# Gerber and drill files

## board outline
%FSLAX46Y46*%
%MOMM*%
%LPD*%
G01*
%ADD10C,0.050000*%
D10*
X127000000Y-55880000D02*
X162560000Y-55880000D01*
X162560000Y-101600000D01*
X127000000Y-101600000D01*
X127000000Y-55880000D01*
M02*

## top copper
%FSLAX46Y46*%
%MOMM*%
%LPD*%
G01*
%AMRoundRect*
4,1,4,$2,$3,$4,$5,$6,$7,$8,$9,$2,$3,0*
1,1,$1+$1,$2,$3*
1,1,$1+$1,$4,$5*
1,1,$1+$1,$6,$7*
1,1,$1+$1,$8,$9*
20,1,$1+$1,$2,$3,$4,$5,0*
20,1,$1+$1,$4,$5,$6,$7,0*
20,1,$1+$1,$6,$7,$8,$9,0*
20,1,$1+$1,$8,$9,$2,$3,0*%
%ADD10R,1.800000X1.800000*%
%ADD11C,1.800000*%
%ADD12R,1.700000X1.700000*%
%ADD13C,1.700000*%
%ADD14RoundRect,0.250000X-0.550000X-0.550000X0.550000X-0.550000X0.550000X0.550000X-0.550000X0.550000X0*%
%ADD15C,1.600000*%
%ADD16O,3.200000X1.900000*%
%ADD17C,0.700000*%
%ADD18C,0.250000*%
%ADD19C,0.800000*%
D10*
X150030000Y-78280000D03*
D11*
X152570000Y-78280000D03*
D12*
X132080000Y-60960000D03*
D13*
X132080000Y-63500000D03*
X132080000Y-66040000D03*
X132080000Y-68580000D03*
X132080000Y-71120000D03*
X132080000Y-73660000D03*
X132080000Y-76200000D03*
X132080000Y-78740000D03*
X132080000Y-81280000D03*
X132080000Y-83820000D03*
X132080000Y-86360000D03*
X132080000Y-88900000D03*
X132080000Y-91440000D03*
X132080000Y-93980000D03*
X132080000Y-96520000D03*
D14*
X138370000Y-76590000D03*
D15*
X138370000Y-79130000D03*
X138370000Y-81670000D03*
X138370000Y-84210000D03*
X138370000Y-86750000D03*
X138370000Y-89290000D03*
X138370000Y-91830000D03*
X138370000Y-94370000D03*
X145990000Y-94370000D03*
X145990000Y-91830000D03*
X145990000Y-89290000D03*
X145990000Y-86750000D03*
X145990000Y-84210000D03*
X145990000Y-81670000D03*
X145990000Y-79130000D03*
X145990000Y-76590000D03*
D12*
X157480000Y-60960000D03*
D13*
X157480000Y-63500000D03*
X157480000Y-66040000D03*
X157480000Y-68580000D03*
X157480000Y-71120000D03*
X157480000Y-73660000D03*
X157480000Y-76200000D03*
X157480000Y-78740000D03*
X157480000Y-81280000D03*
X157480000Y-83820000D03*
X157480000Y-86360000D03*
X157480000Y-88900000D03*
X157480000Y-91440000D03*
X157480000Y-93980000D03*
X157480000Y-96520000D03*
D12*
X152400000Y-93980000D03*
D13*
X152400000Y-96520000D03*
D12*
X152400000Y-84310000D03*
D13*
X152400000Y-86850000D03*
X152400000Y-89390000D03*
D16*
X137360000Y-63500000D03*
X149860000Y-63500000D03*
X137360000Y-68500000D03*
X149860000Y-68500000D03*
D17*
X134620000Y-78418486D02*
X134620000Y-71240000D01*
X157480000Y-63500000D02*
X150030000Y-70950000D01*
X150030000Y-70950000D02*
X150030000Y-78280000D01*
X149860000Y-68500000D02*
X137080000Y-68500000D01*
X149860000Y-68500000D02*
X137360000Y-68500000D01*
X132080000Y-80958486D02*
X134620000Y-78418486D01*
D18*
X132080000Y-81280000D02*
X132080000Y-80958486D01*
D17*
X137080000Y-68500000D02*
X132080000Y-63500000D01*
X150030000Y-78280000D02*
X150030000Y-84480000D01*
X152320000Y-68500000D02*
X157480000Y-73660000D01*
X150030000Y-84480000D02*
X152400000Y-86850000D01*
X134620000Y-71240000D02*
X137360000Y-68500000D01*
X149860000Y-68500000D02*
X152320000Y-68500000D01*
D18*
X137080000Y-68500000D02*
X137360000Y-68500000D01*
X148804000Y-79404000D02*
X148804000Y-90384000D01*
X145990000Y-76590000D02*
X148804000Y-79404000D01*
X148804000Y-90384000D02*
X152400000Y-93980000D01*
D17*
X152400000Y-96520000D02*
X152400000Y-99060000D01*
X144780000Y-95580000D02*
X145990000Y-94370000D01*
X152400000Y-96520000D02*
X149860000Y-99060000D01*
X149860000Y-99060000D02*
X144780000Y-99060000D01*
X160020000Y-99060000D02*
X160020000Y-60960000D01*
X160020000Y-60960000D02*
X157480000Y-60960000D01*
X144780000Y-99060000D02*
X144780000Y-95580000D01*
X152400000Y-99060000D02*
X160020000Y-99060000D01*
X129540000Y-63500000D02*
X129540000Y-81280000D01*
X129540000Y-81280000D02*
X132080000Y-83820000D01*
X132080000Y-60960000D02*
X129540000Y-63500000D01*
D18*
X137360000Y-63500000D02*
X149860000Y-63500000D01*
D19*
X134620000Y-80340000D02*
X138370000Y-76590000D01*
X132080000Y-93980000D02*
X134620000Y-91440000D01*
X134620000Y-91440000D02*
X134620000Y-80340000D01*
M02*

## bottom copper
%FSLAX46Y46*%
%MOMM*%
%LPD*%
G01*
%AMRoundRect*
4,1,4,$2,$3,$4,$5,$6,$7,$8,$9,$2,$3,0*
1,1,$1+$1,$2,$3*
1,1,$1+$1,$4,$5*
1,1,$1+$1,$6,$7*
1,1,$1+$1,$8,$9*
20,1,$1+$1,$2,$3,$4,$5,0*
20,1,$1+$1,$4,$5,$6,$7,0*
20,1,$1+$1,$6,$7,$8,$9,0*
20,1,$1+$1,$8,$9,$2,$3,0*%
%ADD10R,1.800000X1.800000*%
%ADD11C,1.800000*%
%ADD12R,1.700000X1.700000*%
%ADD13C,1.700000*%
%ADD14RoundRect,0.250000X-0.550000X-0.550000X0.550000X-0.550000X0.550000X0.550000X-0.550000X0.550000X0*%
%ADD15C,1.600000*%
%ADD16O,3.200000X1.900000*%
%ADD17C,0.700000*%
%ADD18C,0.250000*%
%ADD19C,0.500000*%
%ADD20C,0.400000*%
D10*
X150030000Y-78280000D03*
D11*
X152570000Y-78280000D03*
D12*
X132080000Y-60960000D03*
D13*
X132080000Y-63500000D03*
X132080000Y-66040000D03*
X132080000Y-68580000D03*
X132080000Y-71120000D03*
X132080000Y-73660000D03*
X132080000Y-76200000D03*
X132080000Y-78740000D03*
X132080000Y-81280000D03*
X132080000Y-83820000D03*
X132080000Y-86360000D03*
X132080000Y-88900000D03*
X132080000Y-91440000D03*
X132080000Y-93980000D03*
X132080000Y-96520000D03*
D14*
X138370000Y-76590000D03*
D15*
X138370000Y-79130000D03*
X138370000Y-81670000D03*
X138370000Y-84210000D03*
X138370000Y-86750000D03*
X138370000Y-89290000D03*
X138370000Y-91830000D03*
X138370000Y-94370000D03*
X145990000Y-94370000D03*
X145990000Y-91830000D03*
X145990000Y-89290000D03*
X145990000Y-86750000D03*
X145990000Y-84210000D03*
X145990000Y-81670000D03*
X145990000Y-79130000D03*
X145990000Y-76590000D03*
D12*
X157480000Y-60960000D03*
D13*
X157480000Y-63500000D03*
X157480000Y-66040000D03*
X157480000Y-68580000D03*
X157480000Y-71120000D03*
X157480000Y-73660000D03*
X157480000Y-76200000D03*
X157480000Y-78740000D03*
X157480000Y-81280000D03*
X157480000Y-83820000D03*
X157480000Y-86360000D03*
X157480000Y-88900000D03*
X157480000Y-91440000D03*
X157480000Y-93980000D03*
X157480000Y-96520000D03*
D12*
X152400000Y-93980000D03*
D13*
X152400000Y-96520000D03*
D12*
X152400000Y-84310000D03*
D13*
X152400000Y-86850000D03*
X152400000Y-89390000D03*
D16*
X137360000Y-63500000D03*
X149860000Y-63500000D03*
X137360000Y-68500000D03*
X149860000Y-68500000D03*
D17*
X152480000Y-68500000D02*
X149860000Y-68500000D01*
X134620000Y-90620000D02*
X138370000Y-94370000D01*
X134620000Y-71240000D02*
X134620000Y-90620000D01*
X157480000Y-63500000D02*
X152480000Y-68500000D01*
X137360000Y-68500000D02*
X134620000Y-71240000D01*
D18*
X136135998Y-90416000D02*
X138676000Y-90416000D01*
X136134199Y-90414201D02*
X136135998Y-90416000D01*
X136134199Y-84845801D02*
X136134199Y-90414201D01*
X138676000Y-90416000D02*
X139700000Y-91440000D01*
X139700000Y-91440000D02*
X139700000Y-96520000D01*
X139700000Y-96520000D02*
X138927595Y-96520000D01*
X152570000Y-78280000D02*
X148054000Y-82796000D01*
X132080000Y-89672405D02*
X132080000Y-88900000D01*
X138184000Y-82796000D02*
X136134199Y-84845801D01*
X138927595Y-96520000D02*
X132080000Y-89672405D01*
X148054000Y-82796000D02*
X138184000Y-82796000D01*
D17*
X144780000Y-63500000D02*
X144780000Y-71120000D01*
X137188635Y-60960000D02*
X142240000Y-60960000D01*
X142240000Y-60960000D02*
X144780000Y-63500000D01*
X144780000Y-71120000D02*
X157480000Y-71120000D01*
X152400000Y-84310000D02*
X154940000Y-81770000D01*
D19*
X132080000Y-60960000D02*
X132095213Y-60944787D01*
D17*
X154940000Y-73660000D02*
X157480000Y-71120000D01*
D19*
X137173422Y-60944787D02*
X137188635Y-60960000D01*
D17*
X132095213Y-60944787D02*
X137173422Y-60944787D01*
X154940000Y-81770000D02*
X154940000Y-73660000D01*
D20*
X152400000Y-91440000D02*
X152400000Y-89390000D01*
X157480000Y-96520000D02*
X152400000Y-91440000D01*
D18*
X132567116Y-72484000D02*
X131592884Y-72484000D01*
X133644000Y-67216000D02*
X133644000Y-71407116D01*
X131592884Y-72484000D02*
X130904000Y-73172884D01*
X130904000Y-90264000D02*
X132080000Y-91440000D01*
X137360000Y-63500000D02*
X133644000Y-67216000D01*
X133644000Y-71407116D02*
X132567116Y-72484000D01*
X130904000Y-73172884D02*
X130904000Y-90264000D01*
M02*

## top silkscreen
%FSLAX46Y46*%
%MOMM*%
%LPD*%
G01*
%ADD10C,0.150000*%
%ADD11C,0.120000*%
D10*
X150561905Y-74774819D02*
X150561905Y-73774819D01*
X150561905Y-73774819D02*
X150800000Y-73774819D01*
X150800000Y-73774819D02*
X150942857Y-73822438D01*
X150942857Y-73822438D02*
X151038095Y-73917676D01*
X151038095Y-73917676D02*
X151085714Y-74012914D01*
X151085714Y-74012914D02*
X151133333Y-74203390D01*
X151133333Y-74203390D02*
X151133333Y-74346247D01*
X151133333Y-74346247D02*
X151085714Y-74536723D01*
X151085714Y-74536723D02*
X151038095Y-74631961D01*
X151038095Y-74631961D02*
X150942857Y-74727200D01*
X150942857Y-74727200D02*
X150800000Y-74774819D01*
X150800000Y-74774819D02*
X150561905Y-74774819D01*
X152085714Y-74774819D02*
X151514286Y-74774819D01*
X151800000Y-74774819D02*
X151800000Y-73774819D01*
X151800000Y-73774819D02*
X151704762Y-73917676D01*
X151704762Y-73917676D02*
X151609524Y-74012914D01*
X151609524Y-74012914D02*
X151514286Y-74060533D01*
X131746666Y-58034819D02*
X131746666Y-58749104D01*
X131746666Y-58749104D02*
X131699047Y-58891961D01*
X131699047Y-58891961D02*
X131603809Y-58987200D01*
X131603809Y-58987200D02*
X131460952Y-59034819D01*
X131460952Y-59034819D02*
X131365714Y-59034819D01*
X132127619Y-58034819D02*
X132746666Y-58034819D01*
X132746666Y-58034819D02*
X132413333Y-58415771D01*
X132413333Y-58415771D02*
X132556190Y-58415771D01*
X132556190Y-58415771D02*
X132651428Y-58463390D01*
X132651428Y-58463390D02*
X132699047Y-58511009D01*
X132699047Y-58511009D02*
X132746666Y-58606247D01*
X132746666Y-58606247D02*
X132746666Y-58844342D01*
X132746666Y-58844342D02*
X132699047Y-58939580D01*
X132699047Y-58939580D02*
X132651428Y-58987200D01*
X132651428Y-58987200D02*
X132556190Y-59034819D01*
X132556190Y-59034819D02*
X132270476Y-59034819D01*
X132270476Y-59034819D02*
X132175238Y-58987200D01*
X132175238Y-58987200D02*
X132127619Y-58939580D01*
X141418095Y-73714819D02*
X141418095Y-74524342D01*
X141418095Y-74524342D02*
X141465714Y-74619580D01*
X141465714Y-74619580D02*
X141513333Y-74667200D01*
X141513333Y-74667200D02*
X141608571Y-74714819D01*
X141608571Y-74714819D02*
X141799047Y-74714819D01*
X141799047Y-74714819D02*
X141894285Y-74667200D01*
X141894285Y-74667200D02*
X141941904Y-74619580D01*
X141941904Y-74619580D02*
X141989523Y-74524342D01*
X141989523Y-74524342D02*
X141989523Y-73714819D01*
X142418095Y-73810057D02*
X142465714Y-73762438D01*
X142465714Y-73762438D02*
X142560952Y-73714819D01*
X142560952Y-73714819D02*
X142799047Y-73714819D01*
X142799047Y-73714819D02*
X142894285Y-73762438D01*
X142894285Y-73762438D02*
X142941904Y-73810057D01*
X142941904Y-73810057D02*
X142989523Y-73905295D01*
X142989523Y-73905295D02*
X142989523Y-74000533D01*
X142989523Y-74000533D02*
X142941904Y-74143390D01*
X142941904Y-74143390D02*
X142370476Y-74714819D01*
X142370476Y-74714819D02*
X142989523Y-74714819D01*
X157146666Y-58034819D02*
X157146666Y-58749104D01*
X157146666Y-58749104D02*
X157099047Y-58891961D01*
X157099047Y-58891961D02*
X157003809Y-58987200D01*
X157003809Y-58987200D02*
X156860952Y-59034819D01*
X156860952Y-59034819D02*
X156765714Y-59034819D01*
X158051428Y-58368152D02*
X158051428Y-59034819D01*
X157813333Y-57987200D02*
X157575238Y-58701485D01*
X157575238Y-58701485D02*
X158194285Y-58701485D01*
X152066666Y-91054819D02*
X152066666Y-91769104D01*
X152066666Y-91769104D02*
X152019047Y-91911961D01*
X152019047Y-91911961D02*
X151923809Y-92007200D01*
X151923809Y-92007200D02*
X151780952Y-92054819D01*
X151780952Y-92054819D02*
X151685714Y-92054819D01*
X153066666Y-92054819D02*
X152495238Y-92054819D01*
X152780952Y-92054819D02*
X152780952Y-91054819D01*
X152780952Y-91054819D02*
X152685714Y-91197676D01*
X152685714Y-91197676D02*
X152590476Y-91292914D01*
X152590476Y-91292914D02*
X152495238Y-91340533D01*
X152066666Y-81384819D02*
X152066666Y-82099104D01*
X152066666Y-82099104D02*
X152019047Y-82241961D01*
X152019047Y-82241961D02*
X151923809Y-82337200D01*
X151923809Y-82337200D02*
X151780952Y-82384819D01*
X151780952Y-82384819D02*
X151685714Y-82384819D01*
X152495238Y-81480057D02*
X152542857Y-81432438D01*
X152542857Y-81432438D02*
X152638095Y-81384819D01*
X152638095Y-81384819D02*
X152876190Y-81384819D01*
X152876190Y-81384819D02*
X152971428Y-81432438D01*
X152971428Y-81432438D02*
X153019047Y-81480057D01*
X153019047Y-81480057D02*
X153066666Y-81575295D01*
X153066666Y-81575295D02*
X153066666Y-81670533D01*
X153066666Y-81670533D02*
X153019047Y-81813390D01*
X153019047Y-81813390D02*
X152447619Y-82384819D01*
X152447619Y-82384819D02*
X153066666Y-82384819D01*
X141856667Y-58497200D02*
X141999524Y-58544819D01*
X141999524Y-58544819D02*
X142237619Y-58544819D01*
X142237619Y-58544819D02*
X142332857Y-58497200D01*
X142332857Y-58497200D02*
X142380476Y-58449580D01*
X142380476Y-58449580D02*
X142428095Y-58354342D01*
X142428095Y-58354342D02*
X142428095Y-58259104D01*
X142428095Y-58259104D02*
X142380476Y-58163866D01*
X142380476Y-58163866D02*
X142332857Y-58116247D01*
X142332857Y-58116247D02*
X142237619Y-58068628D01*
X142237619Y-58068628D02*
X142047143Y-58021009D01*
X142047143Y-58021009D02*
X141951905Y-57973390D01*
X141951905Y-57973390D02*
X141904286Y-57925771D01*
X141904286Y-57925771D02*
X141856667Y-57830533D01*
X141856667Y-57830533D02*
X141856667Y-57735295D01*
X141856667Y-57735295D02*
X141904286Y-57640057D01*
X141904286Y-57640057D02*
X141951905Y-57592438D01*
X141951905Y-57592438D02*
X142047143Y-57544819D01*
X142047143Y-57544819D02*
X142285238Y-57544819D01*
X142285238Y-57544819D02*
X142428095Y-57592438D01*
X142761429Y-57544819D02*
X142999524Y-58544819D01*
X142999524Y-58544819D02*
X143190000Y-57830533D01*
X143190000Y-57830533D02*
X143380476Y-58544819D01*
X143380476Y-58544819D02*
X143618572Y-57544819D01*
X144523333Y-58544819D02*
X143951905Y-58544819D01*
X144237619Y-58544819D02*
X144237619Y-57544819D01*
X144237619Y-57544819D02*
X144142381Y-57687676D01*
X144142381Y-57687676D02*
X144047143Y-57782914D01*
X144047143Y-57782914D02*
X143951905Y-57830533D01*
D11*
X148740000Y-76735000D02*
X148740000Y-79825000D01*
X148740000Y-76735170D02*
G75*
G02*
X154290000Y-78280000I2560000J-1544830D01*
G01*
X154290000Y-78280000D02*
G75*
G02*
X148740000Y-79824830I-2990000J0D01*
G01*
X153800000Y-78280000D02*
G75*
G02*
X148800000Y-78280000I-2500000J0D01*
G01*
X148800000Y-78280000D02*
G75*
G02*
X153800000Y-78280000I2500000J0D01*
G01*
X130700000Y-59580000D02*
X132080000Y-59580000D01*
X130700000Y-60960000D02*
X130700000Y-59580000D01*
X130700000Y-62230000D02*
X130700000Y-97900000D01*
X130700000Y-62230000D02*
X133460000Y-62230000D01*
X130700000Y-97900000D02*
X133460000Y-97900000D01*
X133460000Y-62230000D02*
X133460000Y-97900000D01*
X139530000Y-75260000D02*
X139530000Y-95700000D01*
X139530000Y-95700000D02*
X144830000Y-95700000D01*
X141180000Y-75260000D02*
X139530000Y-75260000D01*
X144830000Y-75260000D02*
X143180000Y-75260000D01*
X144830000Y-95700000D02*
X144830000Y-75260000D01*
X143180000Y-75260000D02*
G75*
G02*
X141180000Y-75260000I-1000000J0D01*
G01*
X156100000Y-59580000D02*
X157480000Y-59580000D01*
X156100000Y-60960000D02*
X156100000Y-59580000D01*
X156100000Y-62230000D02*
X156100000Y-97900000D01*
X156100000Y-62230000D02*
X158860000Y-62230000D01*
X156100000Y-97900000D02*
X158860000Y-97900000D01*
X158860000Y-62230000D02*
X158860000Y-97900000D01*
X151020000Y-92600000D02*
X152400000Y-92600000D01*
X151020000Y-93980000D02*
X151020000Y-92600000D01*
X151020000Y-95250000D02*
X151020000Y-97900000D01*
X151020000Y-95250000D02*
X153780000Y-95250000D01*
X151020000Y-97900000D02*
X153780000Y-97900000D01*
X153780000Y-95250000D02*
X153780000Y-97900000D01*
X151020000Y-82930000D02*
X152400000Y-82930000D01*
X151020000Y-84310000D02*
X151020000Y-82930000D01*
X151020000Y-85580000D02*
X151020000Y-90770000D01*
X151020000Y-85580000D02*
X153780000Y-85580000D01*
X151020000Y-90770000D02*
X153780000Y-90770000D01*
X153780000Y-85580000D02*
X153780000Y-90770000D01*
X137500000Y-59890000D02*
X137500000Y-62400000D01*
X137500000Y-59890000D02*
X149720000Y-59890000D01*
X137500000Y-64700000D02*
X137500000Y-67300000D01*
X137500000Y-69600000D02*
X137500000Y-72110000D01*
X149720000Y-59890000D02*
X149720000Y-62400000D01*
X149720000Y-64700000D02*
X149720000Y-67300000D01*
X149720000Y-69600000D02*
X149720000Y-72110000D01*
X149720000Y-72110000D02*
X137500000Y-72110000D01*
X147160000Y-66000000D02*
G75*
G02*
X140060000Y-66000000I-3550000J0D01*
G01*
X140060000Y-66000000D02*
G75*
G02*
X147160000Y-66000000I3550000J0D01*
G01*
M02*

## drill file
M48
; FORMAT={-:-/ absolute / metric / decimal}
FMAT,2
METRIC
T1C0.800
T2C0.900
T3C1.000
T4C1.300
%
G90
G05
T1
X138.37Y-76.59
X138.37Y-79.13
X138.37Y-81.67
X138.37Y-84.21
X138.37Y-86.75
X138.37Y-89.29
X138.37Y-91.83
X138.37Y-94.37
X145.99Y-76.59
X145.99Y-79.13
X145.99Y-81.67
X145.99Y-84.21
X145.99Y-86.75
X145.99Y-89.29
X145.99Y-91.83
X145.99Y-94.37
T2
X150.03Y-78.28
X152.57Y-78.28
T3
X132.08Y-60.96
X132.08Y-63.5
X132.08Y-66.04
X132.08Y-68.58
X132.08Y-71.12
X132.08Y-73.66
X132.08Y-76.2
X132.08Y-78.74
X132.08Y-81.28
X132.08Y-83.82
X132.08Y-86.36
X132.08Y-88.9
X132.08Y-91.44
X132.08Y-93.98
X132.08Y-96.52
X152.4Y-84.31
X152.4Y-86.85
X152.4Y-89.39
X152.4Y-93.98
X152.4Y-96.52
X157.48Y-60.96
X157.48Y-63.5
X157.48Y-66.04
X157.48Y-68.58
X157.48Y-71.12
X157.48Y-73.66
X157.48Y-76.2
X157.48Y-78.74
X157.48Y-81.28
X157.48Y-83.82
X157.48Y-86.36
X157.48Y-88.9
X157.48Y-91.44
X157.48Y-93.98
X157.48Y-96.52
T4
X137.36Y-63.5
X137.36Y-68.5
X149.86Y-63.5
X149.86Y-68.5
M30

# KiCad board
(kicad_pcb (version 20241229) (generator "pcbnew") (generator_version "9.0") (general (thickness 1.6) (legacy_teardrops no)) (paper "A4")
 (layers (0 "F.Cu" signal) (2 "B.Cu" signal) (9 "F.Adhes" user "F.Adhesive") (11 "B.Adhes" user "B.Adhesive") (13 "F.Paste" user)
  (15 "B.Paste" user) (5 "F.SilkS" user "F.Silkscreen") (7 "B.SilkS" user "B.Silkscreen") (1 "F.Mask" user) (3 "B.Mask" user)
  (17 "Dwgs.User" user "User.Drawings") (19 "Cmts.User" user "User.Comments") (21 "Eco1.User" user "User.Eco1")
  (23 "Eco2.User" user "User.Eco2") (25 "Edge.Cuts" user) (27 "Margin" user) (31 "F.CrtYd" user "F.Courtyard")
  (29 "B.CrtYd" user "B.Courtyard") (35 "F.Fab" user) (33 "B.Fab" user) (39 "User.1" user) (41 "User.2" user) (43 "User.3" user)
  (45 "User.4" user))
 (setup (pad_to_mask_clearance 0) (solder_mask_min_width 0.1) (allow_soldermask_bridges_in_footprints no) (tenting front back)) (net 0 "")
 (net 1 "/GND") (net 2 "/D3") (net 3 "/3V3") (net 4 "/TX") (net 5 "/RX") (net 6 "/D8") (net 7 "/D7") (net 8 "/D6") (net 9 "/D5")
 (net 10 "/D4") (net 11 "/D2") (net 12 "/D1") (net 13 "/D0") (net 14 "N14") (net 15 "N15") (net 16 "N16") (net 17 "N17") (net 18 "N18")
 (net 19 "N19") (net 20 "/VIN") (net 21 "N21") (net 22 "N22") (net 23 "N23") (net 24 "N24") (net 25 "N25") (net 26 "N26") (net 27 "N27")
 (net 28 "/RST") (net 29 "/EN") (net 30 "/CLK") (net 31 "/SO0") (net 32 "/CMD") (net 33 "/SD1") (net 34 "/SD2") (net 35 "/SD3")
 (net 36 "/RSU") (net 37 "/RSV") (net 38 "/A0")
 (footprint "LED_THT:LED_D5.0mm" (layer "F.Cu") (at 150.03 78.28)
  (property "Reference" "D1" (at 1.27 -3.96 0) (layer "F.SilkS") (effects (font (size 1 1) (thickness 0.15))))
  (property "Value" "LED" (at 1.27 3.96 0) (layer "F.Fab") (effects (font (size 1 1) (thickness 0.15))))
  (fp_line (start -1.29 -1.545) (end -1.29 1.545) (stroke (width 0.12) (type solid)) (layer "F.SilkS"))
  (fp_arc (start -1.29 -1.54483) (mid 2.071779 -2.880495) (end 4.26 0) (stroke (width 0.12) (type solid)) (layer "F.SilkS"))
  (fp_arc (start 4.26 0) (mid 2.071779 2.880495) (end -1.29 1.54483) (stroke (width 0.12) (type solid)) (layer "F.SilkS"))
  (fp_circle (center 1.27 0) (end 3.77 0) (stroke (width 0.12) (type solid)) (fill no) (layer "F.SilkS"))
  (pad "1" thru_hole rect (at 0 0) (size 1.8 1.8) (drill 0.9) (layers "*.Cu" "*.Mask") (remove_unused_layers no) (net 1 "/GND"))
  (pad "2" thru_hole circle (at 2.54 0) (size 1.8 1.8) (drill 0.9) (layers "*.Cu" "*.Mask") (remove_unused_layers no) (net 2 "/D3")))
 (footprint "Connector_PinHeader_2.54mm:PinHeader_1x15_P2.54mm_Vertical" (layer "F.Cu") (at 132.08 60.96)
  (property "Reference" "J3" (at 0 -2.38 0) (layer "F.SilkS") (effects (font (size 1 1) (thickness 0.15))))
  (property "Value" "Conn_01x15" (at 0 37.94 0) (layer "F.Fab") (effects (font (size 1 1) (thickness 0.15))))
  (fp_line (start -1.38 -1.38) (end 0 -1.38) (stroke (width 0.12) (type solid)) (layer "F.SilkS"))
  (fp_line (start -1.38 0) (end -1.38 -1.38) (stroke (width 0.12) (type solid)) (layer "F.SilkS"))
  (fp_line (start -1.38 1.27) (end -1.38 36.94) (stroke (width 0.12) (type solid)) (layer "F.SilkS"))
  (fp_line (start -1.38 1.27) (end 1.38 1.27) (stroke (width 0.12) (type solid)) (layer "F.SilkS"))
  (fp_line (start -1.38 36.94) (end 1.38 36.94) (stroke (width 0.12) (type solid)) (layer "F.SilkS"))
  (fp_line (start 1.38 1.27) (end 1.38 36.94) (stroke (width 0.12) (type solid)) (layer "F.SilkS"))
  (pad "1" thru_hole rect (at 0 0) (size 1.7 1.7) (drill 1) (layers "*.Cu" "*.Mask") (remove_unused_layers no) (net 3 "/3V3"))
  (pad "2" thru_hole circle (at 0 2.54) (size 1.7 1.7) (drill 1) (layers "*.Cu" "*.Mask") (remove_unused_layers no) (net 1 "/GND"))
  (pad "3" thru_hole circle (at 0 5.08) (size 1.7 1.7) (drill 1) (layers "*.Cu" "*.Mask") (remove_unused_layers no) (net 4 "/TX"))
  (pad "4" thru_hole circle (at 0 7.62) (size 1.7 1.7) (drill 1) (layers "*.Cu" "*.Mask") (remove_unused_layers no) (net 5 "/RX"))
  (pad "5" thru_hole circle (at 0 10.16) (size 1.7 1.7) (drill 1) (layers "*.Cu" "*.Mask") (remove_unused_layers no) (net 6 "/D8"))
  (pad "6" thru_hole circle (at 0 12.7) (size 1.7 1.7) (drill 1) (layers "*.Cu" "*.Mask") (remove_unused_layers no) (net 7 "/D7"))
  (pad "7" thru_hole circle (at 0 15.24) (size 1.7 1.7) (drill 1) (layers "*.Cu" "*.Mask") (remove_unused_layers no) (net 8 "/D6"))
  (pad "8" thru_hole circle (at 0 17.78) (size 1.7 1.7) (drill 1) (layers "*.Cu" "*.Mask") (remove_unused_layers no) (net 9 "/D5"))
  (pad "9" thru_hole circle (at 0 20.32) (size 1.7 1.7) (drill 1) (layers "*.Cu" "*.Mask") (remove_unused_layers no) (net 1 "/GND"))
  (pad "10" thru_hole circle (at 0 22.86) (size 1.7 1.7) (drill 1) (layers "*.Cu" "*.Mask") (remove_unused_layers no) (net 3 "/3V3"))
  (pad "11" thru_hole circle (at 0 25.4) (size 1.7 1.7) (drill 1) (layers "*.Cu" "*.Mask") (remove_unused_layers no) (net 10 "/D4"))
  (pad "12" thru_hole circle (at 0 27.94) (size 1.7 1.7) (drill 1) (layers "*.Cu" "*.Mask") (remove_unused_layers no) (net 2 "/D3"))
  (pad "13" thru_hole circle (at 0 30.48) (size 1.7 1.7) (drill 1) (layers "*.Cu" "*.Mask") (remove_unused_layers no) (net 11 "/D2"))
  (pad "14" thru_hole circle (at 0 33.02) (size 1.7 1.7) (drill 1) (layers "*.Cu" "*.Mask") (remove_unused_layers no) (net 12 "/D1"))
  (pad "15" thru_hole circle (at 0 35.56) (size 1.7 1.7) (drill 1) (layers "*.Cu" "*.Mask") (remove_unused_layers no) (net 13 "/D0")))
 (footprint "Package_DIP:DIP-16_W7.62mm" (layer "F.Cu") (at 138.37 76.59)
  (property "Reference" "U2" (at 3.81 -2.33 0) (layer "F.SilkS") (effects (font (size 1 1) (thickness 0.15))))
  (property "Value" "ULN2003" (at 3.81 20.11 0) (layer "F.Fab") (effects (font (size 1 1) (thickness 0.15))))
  (fp_line (start 1.16 -1.33) (end 1.16 19.11) (stroke (width 0.12) (type solid)) (layer "F.SilkS"))
  (fp_line (start 1.16 19.11) (end 6.46 19.11) (stroke (width 0.12) (type solid)) (layer "F.SilkS"))
  (fp_line (start 2.81 -1.33) (end 1.16 -1.33) (stroke (width 0.12) (type solid)) (layer "F.SilkS"))
  (fp_line (start 6.46 -1.33) (end 4.81 -1.33) (stroke (width 0.12) (type solid)) (layer "F.SilkS"))
  (fp_line (start 6.46 19.11) (end 6.46 -1.33) (stroke (width 0.12) (type solid)) (layer "F.SilkS"))
  (fp_arc (start 4.81 -1.33) (mid 3.81 -0.33) (end 2.81 -1.33) (stroke (width 0.12) (type solid)) (layer "F.SilkS"))
  (pad "1" thru_hole roundrect (at 0 0) (size 1.6 1.6) (drill 0.8) (layers "*.Cu" "*.Mask") (remove_unused_layers no)
   (roundrect_rratio 0.15625) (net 12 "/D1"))
  (pad "2" thru_hole circle (at 0 2.54) (size 1.6 1.6) (drill 0.8) (layers "*.Cu" "*.Mask") (remove_unused_layers no) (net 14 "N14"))
  (pad "3" thru_hole circle (at 0 5.08) (size 1.6 1.6) (drill 0.8) (layers "*.Cu" "*.Mask") (remove_unused_layers no) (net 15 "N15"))
  (pad "4" thru_hole circle (at 0 7.62) (size 1.6 1.6) (drill 0.8) (layers "*.Cu" "*.Mask") (remove_unused_layers no) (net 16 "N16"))
  (pad "5" thru_hole circle (at 0 10.16) (size 1.6 1.6) (drill 0.8) (layers "*.Cu" "*.Mask") (remove_unused_layers no) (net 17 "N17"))
  (pad "6" thru_hole circle (at 0 12.7) (size 1.6 1.6) (drill 0.8) (layers "*.Cu" "*.Mask") (remove_unused_layers no) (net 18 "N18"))
  (pad "7" thru_hole circle (at 0 15.24) (size 1.6 1.6) (drill 0.8) (layers "*.Cu" "*.Mask") (remove_unused_layers no) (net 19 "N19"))
  (pad "8" thru_hole circle (at 0 17.78) (size 1.6 1.6) (drill 0.8) (layers "*.Cu" "*.Mask") (remove_unused_layers no) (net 1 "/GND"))
  (pad "9" thru_hole circle (at 7.62 17.78) (size 1.6 1.6) (drill 0.8) (layers "*.Cu" "*.Mask") (remove_unused_layers no) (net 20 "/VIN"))
  (pad "10" thru_hole circle (at 7.62 15.24) (size 1.6 1.6) (drill 0.8) (layers "*.Cu" "*.Mask") (remove_unused_layers no) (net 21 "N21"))
  (pad "11" thru_hole circle (at 7.62 12.7) (size 1.6 1.6) (drill 0.8) (layers "*.Cu" "*.Mask") (remove_unused_layers no) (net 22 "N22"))
  (pad "12" thru_hole circle (at 7.62 10.16) (size 1.6 1.6) (drill 0.8) (layers "*.Cu" "*.Mask") (remove_unused_layers no) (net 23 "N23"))
  (pad "13" thru_hole circle (at 7.62 7.62) (size 1.6 1.6) (drill 0.8) (layers "*.Cu" "*.Mask") (remove_unused_layers no) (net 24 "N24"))
  (pad "14" thru_hole circle (at 7.62 5.08) (size 1.6 1.6) (drill 0.8) (layers "*.Cu" "*.Mask") (remove_unused_layers no) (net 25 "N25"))
  (pad "15" thru_hole circle (at 7.62 2.54) (size 1.6 1.6) (drill 0.8) (layers "*.Cu" "*.Mask") (remove_unused_layers no) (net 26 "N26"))
  (pad "16" thru_hole circle (at 7.62 0) (size 1.6 1.6) (drill 0.8) (layers "*.Cu" "*.Mask") (remove_unused_layers no) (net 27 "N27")))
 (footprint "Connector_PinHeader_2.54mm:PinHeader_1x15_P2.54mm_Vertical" (layer "F.Cu") (at 157.48 60.96)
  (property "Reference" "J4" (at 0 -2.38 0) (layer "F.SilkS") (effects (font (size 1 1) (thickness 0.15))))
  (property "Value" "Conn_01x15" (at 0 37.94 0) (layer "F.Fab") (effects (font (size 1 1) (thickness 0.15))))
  (fp_line (start -1.38 -1.38) (end 0 -1.38) (stroke (width 0.12) (type solid)) (layer "F.SilkS"))
  (fp_line (start -1.38 0) (end -1.38 -1.38) (stroke (width 0.12) (type solid)) (layer "F.SilkS"))
  (fp_line (start -1.38 1.27) (end -1.38 36.94) (stroke (width 0.12) (type solid)) (layer "F.SilkS"))
  (fp_line (start -1.38 1.27) (end 1.38 1.27) (stroke (width 0.12) (type solid)) (layer "F.SilkS"))
  (fp_line (start -1.38 36.94) (end 1.38 36.94) (stroke (width 0.12) (type solid)) (layer "F.SilkS"))
  (fp_line (start 1.38 1.27) (end 1.38 36.94) (stroke (width 0.12) (type solid)) (layer "F.SilkS"))
  (pad "1" thru_hole rect (at 0 0) (size 1.7 1.7) (drill 1) (layers "*.Cu" "*.Mask") (remove_unused_layers no) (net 20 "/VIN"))
  (pad "2" thru_hole circle (at 0 2.54) (size 1.7 1.7) (drill 1) (layers "*.Cu" "*.Mask") (remove_unused_layers no) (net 1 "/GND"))
  (pad "3" thru_hole circle (at 0 5.08) (size 1.7 1.7) (drill 1) (layers "*.Cu" "*.Mask") (remove_unused_layers no) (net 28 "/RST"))
  (pad "4" thru_hole circle (at 0 7.62) (size 1.7 1.7) (drill 1) (layers "*.Cu" "*.Mask") (remove_unused_layers no) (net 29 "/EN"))
  (pad "5" thru_hole circle (at 0 10.16) (size 1.7 1.7) (drill 1) (layers "*.Cu" "*.Mask") (remove_unused_layers no) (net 3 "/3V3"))
  (pad "6" thru_hole circle (at 0 12.7) (size 1.7 1.7) (drill 1) (layers "*.Cu" "*.Mask") (remove_unused_layers no) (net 1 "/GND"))
  (pad "7" thru_hole circle (at 0 15.24) (size 1.7 1.7) (drill 1) (layers "*.Cu" "*.Mask") (remove_unused_layers no) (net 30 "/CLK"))
  (pad "8" thru_hole circle (at 0 17.78) (size 1.7 1.7) (drill 1) (layers "*.Cu" "*.Mask") (remove_unused_layers no) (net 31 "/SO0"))
  (pad "9" thru_hole circle (at 0 20.32) (size 1.7 1.7) (drill 1) (layers "*.Cu" "*.Mask") (remove_unused_layers no) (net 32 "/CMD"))
  (pad "10" thru_hole circle (at 0 22.86) (size 1.7 1.7) (drill 1) (layers "*.Cu" "*.Mask") (remove_unused_layers no) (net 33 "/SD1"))
  (pad "11" thru_hole circle (at 0 25.4) (size 1.7 1.7) (drill 1) (layers "*.Cu" "*.Mask") (remove_unused_layers no) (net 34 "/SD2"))
  (pad "12" thru_hole circle (at 0 27.94) (size 1.7 1.7) (drill 1) (layers "*.Cu" "*.Mask") (remove_unused_layers no) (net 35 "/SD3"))
  (pad "13" thru_hole circle (at 0 30.48) (size 1.7 1.7) (drill 1) (layers "*.Cu" "*.Mask") (remove_unused_layers no) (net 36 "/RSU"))
  (pad "14" thru_hole circle (at 0 33.02) (size 1.7 1.7) (drill 1) (layers "*.Cu" "*.Mask") (remove_unused_layers no) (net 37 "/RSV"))
  (pad "15" thru_hole circle (at 0 35.56) (size 1.7 1.7) (drill 1) (layers "*.Cu" "*.Mask") (remove_unused_layers no) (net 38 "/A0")))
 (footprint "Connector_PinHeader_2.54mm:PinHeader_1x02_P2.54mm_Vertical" (layer "F.Cu") (at 152.4 93.98)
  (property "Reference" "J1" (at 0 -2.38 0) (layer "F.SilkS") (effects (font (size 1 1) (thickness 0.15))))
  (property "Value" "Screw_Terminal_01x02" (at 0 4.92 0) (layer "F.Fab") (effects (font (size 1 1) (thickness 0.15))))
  (fp_line (start -1.38 -1.38) (end 0 -1.38) (stroke (width 0.12) (type solid)) (layer "F.SilkS"))
  (fp_line (start -1.38 0) (end -1.38 -1.38) (stroke (width 0.12) (type solid)) (layer "F.SilkS"))
  (fp_line (start -1.38 1.27) (end -1.38 3.92) (stroke (width 0.12) (type solid)) (layer "F.SilkS"))
  (fp_line (start -1.38 1.27) (end 1.38 1.27) (stroke (width 0.12) (type solid)) (layer "F.SilkS"))
  (fp_line (start -1.38 3.92) (end 1.38 3.92) (stroke (width 0.12) (type solid)) (layer "F.SilkS"))
  (fp_line (start 1.38 1.27) (end 1.38 3.92) (stroke (width 0.12) (type solid)) (layer "F.SilkS"))
  (pad "1" thru_hole rect (at 0 0) (size 1.7 1.7) (drill 1) (layers "*.Cu" "*.Mask") (remove_unused_layers no) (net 27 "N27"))
  (pad "2" thru_hole circle (at 0 2.54) (size 1.7 1.7) (drill 1) (layers "*.Cu" "*.Mask") (remove_unused_layers no) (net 20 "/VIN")))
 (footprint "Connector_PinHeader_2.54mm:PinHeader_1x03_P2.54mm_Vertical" (layer "F.Cu") (at 152.4 84.31)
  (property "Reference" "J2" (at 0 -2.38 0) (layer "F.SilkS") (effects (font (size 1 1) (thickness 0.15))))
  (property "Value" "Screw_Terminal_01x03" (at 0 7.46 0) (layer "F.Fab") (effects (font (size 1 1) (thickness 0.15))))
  (fp_line (start -1.38 -1.38) (end 0 -1.38) (stroke (width 0.12) (type solid)) (layer "F.SilkS"))
  (fp_line (start -1.38 0) (end -1.38 -1.38) (stroke (width 0.12) (type solid)) (layer "F.SilkS"))
  (fp_line (start -1.38 1.27) (end -1.38 6.46) (stroke (width 0.12) (type solid)) (layer "F.SilkS"))
  (fp_line (start -1.38 1.27) (end 1.38 1.27) (stroke (width 0.12) (type solid)) (layer "F.SilkS"))
  (fp_line (start -1.38 6.46) (end 1.38 6.46) (stroke (width 0.12) (type solid)) (layer "F.SilkS"))
  (fp_line (start 1.38 1.27) (end 1.38 6.46) (stroke (width 0.12) (type solid)) (layer "F.SilkS"))
  (pad "1" thru_hole rect (at 0 0) (size 1.7 1.7) (drill 1) (layers "*.Cu" "*.Mask") (remove_unused_layers no) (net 3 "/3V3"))
  (pad "2" thru_hole circle (at 0 2.54) (size 1.7 1.7) (drill 1) (layers "*.Cu" "*.Mask") (remove_unused_layers no) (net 1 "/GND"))
  (pad "3" thru_hole circle (at 0 5.08) (size 1.7 1.7) (drill 1) (layers "*.Cu" "*.Mask") (remove_unused_layers no) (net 38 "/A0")))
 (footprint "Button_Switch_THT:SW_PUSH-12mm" (layer "F.Cu") (at 137.36 63.5)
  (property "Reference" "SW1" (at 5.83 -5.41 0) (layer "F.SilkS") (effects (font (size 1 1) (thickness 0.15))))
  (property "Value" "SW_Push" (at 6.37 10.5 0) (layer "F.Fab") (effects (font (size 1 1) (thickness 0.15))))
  (fp_line (start 0.14 -3.61) (end 0.14 -1.1) (stroke (width 0.12) (type default)) (layer "F.SilkS"))
  (fp_line (start 0.14 -3.61) (end 12.36 -3.61) (stroke (width 0.12) (type default)) (layer "F.SilkS"))
  (fp_line (start 0.14 1.2) (end 0.14 3.8) (stroke (width 0.12) (type default)) (layer "F.SilkS"))
  (fp_line (start 0.14 6.1) (end 0.14 8.61) (stroke (width 0.12) (type default)) (layer "F.SilkS"))
  (fp_line (start 12.36 -3.61) (end 12.36 -1.1) (stroke (width 0.12) (type default)) (layer "F.SilkS"))
  (fp_line (start 12.36 1.2) (end 12.36 3.8) (stroke (width 0.12) (type default)) (layer "F.SilkS"))
  (fp_line (start 12.36 6.1) (end 12.36 8.61) (stroke (width 0.12) (type default)) (layer "F.SilkS"))
  (fp_line (start 12.36 8.61) (end 0.14 8.61) (stroke (width 0.12) (type default)) (layer "F.SilkS"))
  (fp_circle (center 6.25 2.5) (end 9.8 2.5) (stroke (width 0.12) (type default)) (fill no) (layer "F.SilkS"))
  (pad "1" thru_hole oval (at 0 0) (size 3.2 1.9) (drill 1.3) (layers "*.Cu" "*.Mask") (remove_unused_layers no) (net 11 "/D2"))
  (pad "1" thru_hole oval (at 12.5 0) (size 3.2 1.9) (drill 1.3) (layers "*.Cu" "*.Mask") (remove_unused_layers no) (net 11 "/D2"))
  (pad "2" thru_hole oval (at 0 5) (size 3.2 1.9) (drill 1.3) (layers "*.Cu" "*.Mask") (remove_unused_layers no) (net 1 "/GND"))
  (pad "2" thru_hole oval (at 12.5 5) (size 3.2 1.9) (drill 1.3) (layers "*.Cu" "*.Mask") (remove_unused_layers no) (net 1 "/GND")))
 (gr_rect (start 127 55.88) (end 162.56 101.6) (stroke (width 0.05) (type default)) (fill no) (layer "Edge.Cuts"))
 (segment (start 134.62 78.418486) (end 134.62 71.24) (width 0.7) (layer "F.Cu") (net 1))
 (segment (start 157.48 63.5) (end 150.03 70.95) (width 0.7) (layer "F.Cu") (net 1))
 (segment (start 150.03 70.95) (end 150.03 78.28) (width 0.7) (layer "F.Cu") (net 1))
 (segment (start 149.86 68.5) (end 137.08 68.5) (width 0.7) (layer "F.Cu") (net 1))
 (segment (start 149.86 68.5) (end 137.36 68.5) (width 0.7) (layer "F.Cu") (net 1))
 (segment (start 132.08 80.958486) (end 134.62 78.418486) (width 0.7) (layer "F.Cu") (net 1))
 (segment (start 132.08 81.28) (end 132.08 80.958486) (width 0.25) (layer "F.Cu") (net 1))
 (segment (start 137.08 68.5) (end 132.08 63.5) (width 0.7) (layer "F.Cu") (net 1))
 (segment (start 150.03 78.28) (end 150.03 84.48) (width 0.7) (layer "F.Cu") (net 1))
 (segment (start 152.32 68.5) (end 157.48 73.66) (width 0.7) (layer "F.Cu") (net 1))
 (segment (start 150.03 84.48) (end 152.4 86.85) (width 0.7) (layer "F.Cu") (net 1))
 (segment (start 134.62 71.24) (end 137.36 68.5) (width 0.7) (layer "F.Cu") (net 1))
 (segment (start 149.86 68.5) (end 152.32 68.5) (width 0.7) (layer "F.Cu") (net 1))
 (segment (start 137.08 68.5) (end 137.36 68.5) (width 0.25) (layer "F.Cu") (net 1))
 (segment (start 152.48 68.5) (end 149.86 68.5) (width 0.7) (layer "B.Cu") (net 1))
 (segment (start 134.62 90.62) (end 138.37 94.37) (width 0.7) (layer "B.Cu") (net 1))
 (segment (start 134.62 71.24) (end 134.62 90.62) (width 0.7) (layer "B.Cu") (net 1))
 (segment (start 157.48 63.5) (end 152.48 68.5) (width 0.7) (layer "B.Cu") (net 1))
 (segment (start 137.36 68.5) (end 134.62 71.24) (width 0.7) (layer "B.Cu") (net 1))
 (segment (start 136.135998 90.416) (end 138.676 90.416) (width 0.25) (layer "B.Cu") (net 2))
 (segment (start 136.134199 90.414201) (end 136.135998 90.416) (width 0.25) (layer "B.Cu") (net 2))
 (segment (start 136.134199 84.845801) (end 136.134199 90.414201) (width 0.25) (layer "B.Cu") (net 2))
 (segment (start 138.676 90.416) (end 139.7 91.44) (width 0.25) (layer "B.Cu") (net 2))
 (segment (start 139.7 91.44) (end 139.7 96.52) (width 0.25) (layer "B.Cu") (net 2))
 (segment (start 139.7 96.52) (end 138.927595 96.52) (width 0.25) (layer "B.Cu") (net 2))
 (segment (start 152.57 78.28) (end 148.054 82.796) (width 0.25) (layer "B.Cu") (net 2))
 (segment (start 132.08 89.672405) (end 132.08 88.9) (width 0.25) (layer "B.Cu") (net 2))
 (segment (start 138.184 82.796) (end 136.134199 84.845801) (width 0.25) (layer "B.Cu") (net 2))
 (segment (start 138.927595 96.52) (end 132.08 89.672405) (width 0.25) (layer "B.Cu") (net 2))
 (segment (start 148.054 82.796) (end 138.184 82.796) (width 0.25) (layer "B.Cu") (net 2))
 (segment (start 148.804 79.404) (end 148.804 90.384) (width 0.25) (layer "F.Cu") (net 27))
 (segment (start 145.99 76.59) (end 148.804 79.404) (width 0.25) (layer "F.Cu") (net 27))
 (segment (start 148.804 90.384) (end 152.4 93.98) (width 0.25) (layer "F.Cu") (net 27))
 (segment (start 152.4 96.52) (end 152.4 99.06) (width 0.7) (layer "F.Cu") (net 20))
 (segment (start 144.78 95.58) (end 145.99 94.37) (width 0.7) (layer "F.Cu") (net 20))
 (segment (start 152.4 96.52) (end 149.86 99.06) (width 0.7) (layer "F.Cu") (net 20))
 (segment (start 149.86 99.06) (end 144.78 99.06) (width 0.7) (layer "F.Cu") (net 20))
 (segment (start 160.02 99.06) (end 160.02 60.96) (width 0.7) (layer "F.Cu") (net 20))
 (segment (start 160.02 60.96) (end 157.48 60.96) (width 0.7) (layer "F.Cu") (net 20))
 (segment (start 144.78 99.06) (end 144.78 95.58) (width 0.7) (layer "F.Cu") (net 20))
 (segment (start 152.4 99.06) (end 160.02 99.06) (width 0.7) (layer "F.Cu") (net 20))
 (segment (start 129.54 63.5) (end 129.54 81.28) (width 0.7) (layer "F.Cu") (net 3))
 (segment (start 129.54 81.28) (end 132.08 83.82) (width 0.7) (layer "F.Cu") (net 3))
 (segment (start 132.08 60.96) (end 129.54 63.5) (width 0.7) (layer "F.Cu") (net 3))
 (segment (start 144.78 63.5) (end 144.78 71.12) (width 0.7) (layer "B.Cu") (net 3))
 (segment (start 137.188635 60.96) (end 142.24 60.96) (width 0.7) (layer "B.Cu") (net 3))
 (segment (start 142.24 60.96) (end 144.78 63.5) (width 0.7) (layer "B.Cu") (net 3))
 (segment (start 144.78 71.12) (end 157.48 71.12) (width 0.7) (layer "B.Cu") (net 3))
 (segment (start 152.4 84.31) (end 154.94 81.77) (width 0.7) (layer "B.Cu") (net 3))
 (segment (start 132.08 60.96) (end 132.095213 60.944787) (width 0.5) (layer "B.Cu") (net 3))
 (segment (start 154.94 73.66) (end 157.48 71.12) (width 0.7) (layer "B.Cu") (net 3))
 (segment (start 137.173422 60.944787) (end 137.188635 60.96) (width 0.5) (layer "B.Cu") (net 3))
 (segment (start 132.095213 60.944787) (end 137.173422 60.944787) (width 0.7) (layer "B.Cu") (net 3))
 (segment (start 154.94 81.77) (end 154.94 73.66) (width 0.7) (layer "B.Cu") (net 3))
 (segment (start 152.4 91.44) (end 152.4 89.39) (width 0.4) (layer "B.Cu") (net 38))
 (segment (start 157.48 96.52) (end 152.4 91.44) (width 0.4) (layer "B.Cu") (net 38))
 (segment (start 137.36 63.5) (end 149.86 63.5) (width 0.25) (layer "F.Cu") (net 11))
 (segment (start 132.567116 72.484) (end 131.592884 72.484) (width 0.25) (layer "B.Cu") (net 11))
 (segment (start 133.644 67.216) (end 133.644 71.407116) (width 0.25) (layer "B.Cu") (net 11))
 (segment (start 131.592884 72.484) (end 130.904 73.172884) (width 0.25) (layer "B.Cu") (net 11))
 (segment (start 130.904 90.264) (end 132.08 91.44) (width 0.25) (layer "B.Cu") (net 11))
 (segment (start 137.36 63.5) (end 133.644 67.216) (width 0.25) (layer "B.Cu") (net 11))
 (segment (start 133.644 71.407116) (end 132.567116 72.484) (width 0.25) (layer "B.Cu") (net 11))
 (segment (start 130.904 73.172884) (end 130.904 90.264) (width 0.25) (layer "B.Cu") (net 11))
 (segment (start 134.62 80.34) (end 138.37 76.59) (width 0.8) (layer "F.Cu") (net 12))
 (segment (start 132.08 93.98) (end 134.62 91.44) (width 0.8) (layer "F.Cu") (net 12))
 (segment (start 134.62 91.44) (end 134.62 80.34) (width 0.8) (layer "F.Cu") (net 12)))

